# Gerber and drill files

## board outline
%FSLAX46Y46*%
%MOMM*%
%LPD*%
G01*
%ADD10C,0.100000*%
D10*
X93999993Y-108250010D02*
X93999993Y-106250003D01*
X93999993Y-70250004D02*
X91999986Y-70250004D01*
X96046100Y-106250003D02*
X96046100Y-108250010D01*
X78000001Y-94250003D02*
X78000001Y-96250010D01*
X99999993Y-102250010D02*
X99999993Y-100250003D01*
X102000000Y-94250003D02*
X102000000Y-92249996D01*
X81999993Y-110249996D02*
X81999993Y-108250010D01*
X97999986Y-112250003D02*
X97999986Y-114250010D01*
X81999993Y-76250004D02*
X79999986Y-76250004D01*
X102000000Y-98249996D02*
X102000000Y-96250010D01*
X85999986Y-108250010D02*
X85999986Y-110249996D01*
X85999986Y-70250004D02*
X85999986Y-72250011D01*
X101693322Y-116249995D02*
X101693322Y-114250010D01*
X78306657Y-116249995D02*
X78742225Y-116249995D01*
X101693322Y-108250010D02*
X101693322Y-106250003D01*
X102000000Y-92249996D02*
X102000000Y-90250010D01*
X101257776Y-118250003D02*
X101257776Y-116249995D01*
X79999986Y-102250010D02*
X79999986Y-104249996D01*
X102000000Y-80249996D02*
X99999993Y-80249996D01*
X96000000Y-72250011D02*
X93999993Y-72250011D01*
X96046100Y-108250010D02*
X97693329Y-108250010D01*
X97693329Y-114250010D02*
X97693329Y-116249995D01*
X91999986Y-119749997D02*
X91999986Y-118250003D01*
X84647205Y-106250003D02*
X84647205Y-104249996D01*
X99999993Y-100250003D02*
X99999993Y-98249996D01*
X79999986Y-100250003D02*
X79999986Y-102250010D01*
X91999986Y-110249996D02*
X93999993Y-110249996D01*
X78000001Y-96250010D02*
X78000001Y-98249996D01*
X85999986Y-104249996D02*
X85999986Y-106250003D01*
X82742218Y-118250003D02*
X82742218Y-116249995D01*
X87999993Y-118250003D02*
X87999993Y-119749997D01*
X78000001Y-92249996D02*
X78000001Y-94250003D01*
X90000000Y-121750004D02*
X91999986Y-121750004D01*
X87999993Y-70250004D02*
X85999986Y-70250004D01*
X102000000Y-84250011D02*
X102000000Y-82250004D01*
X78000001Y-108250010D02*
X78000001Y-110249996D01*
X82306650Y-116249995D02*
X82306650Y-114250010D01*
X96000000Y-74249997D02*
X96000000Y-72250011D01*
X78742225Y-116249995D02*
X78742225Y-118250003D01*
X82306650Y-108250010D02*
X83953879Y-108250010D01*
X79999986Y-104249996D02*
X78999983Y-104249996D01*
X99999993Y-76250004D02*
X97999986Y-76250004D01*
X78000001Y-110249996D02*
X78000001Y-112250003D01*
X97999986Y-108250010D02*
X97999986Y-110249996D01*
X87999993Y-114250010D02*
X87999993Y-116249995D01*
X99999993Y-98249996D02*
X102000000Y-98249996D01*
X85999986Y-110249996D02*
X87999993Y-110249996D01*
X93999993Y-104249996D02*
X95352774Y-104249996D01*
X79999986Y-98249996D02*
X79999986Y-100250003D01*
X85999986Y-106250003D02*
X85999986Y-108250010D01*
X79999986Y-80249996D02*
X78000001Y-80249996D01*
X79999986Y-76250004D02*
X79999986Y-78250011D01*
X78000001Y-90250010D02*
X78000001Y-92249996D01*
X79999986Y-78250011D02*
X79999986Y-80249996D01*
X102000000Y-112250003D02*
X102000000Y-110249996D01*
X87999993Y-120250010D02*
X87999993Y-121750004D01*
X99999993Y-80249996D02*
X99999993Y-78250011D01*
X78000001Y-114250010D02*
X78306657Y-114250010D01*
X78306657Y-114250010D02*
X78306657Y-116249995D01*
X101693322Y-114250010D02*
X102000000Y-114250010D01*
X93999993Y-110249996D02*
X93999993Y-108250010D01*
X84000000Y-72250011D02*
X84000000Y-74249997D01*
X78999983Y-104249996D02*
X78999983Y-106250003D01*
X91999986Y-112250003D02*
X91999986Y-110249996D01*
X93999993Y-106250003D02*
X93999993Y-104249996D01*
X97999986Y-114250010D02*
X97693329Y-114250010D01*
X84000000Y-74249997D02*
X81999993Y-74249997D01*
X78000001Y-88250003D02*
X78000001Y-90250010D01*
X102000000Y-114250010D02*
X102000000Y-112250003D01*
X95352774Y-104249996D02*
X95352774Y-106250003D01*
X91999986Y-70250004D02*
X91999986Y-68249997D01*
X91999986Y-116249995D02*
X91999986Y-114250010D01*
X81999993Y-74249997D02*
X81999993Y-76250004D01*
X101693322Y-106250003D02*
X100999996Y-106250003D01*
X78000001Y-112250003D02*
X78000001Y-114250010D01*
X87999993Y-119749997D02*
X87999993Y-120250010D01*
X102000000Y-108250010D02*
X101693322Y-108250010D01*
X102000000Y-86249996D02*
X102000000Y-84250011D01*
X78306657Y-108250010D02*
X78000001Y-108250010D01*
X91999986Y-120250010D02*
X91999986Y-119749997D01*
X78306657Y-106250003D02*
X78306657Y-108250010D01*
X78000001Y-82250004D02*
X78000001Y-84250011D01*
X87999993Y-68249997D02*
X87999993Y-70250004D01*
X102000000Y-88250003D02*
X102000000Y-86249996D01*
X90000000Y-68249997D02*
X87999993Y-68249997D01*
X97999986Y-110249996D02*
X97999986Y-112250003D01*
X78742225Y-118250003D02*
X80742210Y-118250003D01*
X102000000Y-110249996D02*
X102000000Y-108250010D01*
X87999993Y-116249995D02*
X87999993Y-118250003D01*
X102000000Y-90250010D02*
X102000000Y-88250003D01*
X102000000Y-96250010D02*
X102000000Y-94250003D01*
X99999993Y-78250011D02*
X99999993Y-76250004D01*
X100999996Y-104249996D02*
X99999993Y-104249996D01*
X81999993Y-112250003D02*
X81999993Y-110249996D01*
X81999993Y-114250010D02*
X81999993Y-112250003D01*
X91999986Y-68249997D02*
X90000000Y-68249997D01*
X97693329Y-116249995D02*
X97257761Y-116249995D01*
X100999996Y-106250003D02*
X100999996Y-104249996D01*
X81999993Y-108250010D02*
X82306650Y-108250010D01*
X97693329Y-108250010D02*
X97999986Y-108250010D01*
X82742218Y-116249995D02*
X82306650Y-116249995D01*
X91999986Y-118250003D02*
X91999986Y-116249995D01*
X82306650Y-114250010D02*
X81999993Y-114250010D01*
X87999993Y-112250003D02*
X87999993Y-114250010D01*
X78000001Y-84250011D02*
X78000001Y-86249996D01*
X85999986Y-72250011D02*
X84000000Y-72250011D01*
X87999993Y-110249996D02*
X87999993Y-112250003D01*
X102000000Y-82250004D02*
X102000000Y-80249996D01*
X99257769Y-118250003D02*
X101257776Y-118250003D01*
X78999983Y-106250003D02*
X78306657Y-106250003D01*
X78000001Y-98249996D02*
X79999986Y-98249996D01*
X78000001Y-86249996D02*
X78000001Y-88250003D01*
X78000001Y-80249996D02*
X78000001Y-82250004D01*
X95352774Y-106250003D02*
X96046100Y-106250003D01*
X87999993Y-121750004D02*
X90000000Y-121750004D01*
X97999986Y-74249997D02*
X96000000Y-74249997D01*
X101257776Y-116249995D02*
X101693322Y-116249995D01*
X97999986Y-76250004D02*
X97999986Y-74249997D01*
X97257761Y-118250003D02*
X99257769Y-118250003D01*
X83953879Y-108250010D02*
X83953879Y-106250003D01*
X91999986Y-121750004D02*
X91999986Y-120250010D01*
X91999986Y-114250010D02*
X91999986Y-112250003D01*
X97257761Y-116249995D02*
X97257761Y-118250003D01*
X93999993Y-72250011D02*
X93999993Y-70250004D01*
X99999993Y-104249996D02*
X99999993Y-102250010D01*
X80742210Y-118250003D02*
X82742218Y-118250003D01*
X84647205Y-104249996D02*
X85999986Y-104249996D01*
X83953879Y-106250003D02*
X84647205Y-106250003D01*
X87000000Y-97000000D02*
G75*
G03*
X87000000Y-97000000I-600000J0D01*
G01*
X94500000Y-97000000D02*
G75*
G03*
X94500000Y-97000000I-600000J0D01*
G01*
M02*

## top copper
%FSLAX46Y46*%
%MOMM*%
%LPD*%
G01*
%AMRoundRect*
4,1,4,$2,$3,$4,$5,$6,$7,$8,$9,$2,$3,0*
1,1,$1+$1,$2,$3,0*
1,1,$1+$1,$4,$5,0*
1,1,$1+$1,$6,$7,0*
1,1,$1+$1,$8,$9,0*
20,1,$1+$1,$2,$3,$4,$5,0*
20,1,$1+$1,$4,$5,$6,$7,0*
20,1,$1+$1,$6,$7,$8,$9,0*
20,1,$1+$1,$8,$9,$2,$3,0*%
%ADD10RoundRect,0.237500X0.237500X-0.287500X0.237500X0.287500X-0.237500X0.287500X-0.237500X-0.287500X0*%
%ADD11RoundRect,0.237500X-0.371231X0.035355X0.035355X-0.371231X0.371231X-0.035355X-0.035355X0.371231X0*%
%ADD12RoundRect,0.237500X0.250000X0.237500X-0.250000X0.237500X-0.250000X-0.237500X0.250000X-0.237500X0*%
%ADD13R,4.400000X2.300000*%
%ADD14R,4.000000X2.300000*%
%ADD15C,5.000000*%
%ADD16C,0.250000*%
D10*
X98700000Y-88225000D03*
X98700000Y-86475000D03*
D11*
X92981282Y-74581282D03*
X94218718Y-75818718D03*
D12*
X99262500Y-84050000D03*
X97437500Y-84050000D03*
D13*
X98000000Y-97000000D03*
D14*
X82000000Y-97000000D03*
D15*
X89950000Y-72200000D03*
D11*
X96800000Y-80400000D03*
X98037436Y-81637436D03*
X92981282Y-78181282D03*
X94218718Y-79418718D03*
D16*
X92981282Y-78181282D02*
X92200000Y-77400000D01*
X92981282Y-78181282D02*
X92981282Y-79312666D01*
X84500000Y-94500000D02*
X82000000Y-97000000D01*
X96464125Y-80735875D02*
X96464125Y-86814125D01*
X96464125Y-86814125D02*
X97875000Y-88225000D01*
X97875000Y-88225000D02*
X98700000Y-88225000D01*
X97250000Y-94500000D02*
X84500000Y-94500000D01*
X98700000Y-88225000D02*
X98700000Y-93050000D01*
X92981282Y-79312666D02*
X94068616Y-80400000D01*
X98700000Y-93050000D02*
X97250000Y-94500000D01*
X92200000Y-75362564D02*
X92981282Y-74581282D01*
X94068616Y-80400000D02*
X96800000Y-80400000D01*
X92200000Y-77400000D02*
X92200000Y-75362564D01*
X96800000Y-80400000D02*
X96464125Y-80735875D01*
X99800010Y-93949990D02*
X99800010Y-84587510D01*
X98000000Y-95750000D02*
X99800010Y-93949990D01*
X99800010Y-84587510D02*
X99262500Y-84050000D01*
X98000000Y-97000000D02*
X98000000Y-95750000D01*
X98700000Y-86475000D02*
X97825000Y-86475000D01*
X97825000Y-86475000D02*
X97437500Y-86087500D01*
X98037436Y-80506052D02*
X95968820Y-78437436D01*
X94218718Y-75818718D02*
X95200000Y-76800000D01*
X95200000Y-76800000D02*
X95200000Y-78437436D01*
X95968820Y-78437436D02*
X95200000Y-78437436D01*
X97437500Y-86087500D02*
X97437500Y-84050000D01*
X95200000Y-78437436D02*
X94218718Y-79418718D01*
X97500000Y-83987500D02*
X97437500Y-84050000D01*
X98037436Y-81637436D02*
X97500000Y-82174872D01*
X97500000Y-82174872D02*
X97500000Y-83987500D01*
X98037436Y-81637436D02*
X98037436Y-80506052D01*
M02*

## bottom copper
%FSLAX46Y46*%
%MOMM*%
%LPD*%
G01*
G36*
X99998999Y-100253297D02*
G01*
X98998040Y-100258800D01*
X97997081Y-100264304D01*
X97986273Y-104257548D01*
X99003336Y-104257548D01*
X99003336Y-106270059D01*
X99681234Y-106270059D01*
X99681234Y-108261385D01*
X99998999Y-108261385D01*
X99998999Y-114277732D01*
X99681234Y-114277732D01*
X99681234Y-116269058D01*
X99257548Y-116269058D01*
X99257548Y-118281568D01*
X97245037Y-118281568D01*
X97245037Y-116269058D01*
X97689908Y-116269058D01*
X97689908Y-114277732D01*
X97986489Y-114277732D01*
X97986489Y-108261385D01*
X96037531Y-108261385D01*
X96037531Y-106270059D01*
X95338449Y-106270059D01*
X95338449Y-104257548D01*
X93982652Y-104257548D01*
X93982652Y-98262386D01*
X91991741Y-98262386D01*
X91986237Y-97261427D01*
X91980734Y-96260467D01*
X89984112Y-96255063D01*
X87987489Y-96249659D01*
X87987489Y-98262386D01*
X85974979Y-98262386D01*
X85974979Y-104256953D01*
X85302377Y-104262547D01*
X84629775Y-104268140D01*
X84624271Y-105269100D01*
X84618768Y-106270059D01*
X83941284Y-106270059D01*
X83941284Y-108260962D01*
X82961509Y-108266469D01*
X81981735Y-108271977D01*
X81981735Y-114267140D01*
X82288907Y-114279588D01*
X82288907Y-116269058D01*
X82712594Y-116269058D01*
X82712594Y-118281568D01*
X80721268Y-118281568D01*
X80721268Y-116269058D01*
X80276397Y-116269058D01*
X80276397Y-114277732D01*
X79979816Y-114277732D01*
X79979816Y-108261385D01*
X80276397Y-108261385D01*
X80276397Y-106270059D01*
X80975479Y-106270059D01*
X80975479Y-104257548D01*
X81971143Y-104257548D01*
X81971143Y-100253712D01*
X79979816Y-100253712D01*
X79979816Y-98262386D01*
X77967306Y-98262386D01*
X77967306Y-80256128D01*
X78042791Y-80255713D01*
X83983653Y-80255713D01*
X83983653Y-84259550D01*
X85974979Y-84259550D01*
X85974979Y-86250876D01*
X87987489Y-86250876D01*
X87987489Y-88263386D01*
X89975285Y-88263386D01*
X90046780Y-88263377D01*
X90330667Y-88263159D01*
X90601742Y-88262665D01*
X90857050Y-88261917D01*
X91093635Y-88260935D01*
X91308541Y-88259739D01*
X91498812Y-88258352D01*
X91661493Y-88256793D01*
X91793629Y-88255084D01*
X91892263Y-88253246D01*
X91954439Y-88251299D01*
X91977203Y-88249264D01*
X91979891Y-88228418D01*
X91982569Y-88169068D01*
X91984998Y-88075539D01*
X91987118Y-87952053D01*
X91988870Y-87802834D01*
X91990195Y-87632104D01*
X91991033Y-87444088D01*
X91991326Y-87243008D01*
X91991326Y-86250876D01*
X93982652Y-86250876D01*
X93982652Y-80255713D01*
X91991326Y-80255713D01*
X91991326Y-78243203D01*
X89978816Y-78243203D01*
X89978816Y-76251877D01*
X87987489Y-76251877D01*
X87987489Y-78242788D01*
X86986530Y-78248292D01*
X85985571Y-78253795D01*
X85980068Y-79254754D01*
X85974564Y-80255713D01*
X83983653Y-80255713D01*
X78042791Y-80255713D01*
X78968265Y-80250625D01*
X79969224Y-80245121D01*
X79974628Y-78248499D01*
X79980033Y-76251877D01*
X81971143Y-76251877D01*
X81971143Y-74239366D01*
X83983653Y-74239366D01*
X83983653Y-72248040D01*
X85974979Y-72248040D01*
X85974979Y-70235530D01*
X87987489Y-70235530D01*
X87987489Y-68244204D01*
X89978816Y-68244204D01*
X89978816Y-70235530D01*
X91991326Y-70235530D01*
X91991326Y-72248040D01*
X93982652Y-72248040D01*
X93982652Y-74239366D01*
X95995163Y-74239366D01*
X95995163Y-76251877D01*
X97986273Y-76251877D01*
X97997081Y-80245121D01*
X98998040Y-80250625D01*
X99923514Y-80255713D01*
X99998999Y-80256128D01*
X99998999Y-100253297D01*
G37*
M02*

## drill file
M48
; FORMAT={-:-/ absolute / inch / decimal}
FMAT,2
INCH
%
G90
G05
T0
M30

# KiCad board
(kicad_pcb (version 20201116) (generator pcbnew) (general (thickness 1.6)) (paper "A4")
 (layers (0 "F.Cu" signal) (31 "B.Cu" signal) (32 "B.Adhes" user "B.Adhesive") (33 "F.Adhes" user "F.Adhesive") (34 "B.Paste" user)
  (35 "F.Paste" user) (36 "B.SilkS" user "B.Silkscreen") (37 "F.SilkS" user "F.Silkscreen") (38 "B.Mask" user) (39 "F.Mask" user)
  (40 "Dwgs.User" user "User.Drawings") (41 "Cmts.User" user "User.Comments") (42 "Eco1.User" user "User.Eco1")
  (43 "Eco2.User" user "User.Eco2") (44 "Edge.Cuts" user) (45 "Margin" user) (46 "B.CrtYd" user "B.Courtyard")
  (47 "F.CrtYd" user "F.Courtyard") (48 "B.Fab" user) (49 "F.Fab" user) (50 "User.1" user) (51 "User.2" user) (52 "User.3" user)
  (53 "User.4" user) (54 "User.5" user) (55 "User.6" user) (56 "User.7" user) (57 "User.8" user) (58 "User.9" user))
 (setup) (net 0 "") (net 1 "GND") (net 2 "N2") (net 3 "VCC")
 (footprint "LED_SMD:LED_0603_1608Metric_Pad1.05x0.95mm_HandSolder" (layer "F.Cu") (at 98.7 87.35 90)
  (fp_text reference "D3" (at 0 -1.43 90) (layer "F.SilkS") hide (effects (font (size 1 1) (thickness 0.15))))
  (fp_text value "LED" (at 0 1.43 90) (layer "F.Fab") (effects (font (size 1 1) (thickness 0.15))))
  (pad "1" smd roundrect (at -0.875 0 90) (size 1.05 0.95) (layers "F.Cu" "F.Paste" "F.Mask") (roundrect_rratio 0.25) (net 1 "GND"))
  (pad "2" smd roundrect (at 0.875 0 90) (size 1.05 0.95) (layers "F.Cu" "F.Paste" "F.Mask") (roundrect_rratio 0.25) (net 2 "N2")))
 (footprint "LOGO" (layer "F.Cu") (at 82.05 87.7)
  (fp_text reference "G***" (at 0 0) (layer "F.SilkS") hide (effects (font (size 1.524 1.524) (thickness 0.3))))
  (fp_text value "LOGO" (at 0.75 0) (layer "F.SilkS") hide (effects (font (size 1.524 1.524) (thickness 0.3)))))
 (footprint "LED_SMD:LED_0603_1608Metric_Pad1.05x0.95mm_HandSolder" (layer "F.Cu") (at 93.6 75.2 -45)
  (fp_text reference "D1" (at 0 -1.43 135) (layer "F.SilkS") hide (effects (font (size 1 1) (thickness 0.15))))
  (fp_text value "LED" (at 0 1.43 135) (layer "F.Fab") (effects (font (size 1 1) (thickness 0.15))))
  (pad "1" smd roundrect (at -0.875 0 315) (size 1.05 0.95) (layers "F.Cu" "F.Paste" "F.Mask") (roundrect_rratio 0.25) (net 1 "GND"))
  (pad "2" smd roundrect (at 0.875 0 315) (size 1.05 0.95) (layers "F.Cu" "F.Paste" "F.Mask") (roundrect_rratio 0.25) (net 2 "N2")))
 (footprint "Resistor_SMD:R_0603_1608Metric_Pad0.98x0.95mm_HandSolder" (layer "F.Cu") (at 98.35 84.05 180)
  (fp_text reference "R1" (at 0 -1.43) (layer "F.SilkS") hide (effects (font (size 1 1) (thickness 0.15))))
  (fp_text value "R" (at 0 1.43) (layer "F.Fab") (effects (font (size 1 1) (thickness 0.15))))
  (pad "1" smd roundrect (at -0.9125 0 180) (size 0.975 0.95) (layers "F.Cu" "F.Paste" "F.Mask") (roundrect_rratio 0.25) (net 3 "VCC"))
  (pad "2" smd roundrect (at 0.9125 0 180) (size 0.975 0.95) (layers "F.Cu" "F.Paste" "F.Mask") (roundrect_rratio 0.25) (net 2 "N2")))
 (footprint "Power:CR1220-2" (layer "F.Cu") (at 90 97 90)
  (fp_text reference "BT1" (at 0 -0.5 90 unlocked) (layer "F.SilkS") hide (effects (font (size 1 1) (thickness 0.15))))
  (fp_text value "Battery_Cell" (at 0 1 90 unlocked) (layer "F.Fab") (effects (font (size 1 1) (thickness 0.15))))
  (fp_circle (center 0 -3.6) (end 0.6 -3.6) (layer "Edge.Cuts") (width 0.1) (fill none))
  (fp_circle (center 0 3.9) (end 0.6 3.9) (layer "Edge.Cuts") (width 0.1) (fill none))
  (pad "1" smd rect (at 0 8 90) (size 2.3 4.4) (layers "F.Cu" "F.Paste" "F.Mask") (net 3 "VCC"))
  (pad "2" smd rect (at 0 -8 90) (size 2.3 4) (layers "F.Cu" "F.Paste" "F.Mask") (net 1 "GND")))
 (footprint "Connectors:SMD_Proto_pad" (layer "F.Cu") (at 89.95 72.2)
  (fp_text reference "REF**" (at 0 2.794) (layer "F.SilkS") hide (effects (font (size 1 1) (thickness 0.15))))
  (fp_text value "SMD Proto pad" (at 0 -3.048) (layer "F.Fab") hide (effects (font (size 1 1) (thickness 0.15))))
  (pad "1" smd circle (at 0 0) (size 5 5) (layers "F.Cu" "F.Mask")))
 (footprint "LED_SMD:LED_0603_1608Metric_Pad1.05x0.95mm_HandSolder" (layer "F.Cu") (at 97.418718 81.018718 -45)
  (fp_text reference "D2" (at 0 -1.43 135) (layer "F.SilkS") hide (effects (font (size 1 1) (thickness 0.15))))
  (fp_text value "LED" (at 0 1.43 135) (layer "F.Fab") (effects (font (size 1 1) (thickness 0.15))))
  (pad "1" smd roundrect (at -0.875 0 315) (size 1.05 0.95) (layers "F.Cu" "F.Paste" "F.Mask") (roundrect_rratio 0.25) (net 1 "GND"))
  (pad "2" smd roundrect (at 0.875 0 315) (size 1.05 0.95) (layers "F.Cu" "F.Paste" "F.Mask") (roundrect_rratio 0.25) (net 2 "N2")))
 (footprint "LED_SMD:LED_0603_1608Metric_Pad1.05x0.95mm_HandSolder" (layer "F.Cu") (at 93.6 78.8 -45)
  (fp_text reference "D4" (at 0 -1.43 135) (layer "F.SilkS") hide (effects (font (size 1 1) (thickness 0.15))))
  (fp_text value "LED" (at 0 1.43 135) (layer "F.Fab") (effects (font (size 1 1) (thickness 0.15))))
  (pad "1" smd roundrect (at -0.875 0 315) (size 1.05 0.95) (layers "F.Cu" "F.Paste" "F.Mask") (roundrect_rratio 0.25) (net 1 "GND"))
  (pad "2" smd roundrect (at 0.875 0 315) (size 1.05 0.95) (layers "F.Cu" "F.Paste" "F.Mask") (roundrect_rratio 0.25) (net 2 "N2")))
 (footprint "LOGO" (layer "B.Cu") (at 90 95 180)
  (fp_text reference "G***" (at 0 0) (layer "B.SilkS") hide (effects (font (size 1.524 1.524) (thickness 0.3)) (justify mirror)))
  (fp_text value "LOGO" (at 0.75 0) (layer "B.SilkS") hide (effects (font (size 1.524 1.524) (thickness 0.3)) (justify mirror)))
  (fp_poly
   (pts (xy 2.012511 24.76447) (xy 4.025021 24.76447) (xy 4.025021 22.75196) (xy 6.016347 22.75196) (xy 6.016347 20.760634)
    (xy 8.028857 20.760634) (xy 8.028857 18.748123) (xy 10.019967 18.748123) (xy 10.025372 16.751501) (xy 10.030776 14.754879)
    (xy 11.031735 14.749375) (xy 12.032694 14.743872) (xy 12.032694 -3.262386) (xy 10.020184 -3.262386) (xy 10.020184 -5.253712)
    (xy 8.028857 -5.253712) (xy 8.028857 -9.257548) (xy 9.024521 -9.257548) (xy 9.024521 -11.270059) (xy 9.723603 -11.270059)
    (xy 9.723603 -13.261385) (xy 10.020184 -13.261385) (xy 10.020184 -19.277732) (xy 9.723603 -19.277732) (xy 9.723603 -21.269058)
    (xy 9.278732 -21.269058) (xy 9.278732 -23.281568) (xy 7.287406 -23.281568) (xy 7.287406 -21.269058) (xy 7.711093 -21.269058)
    (xy 7.711093 -19.279588) (xy 8.018265 -19.26714) (xy 8.018265 -13.271977) (xy 7.038491 -13.266469) (xy 6.058716 -13.260962)
    (xy 6.058716 -11.270059) (xy 5.381232 -11.270059) (xy 5.375729 -10.2691) (xy 5.370225 -9.26814) (xy 4.697623 -9.262547)
    (xy 4.025021 -9.256953) (xy 4.025021 -3.262386) (xy 2.012511 -3.262386) (xy 2.012511 -1.249659) (xy 0.015888 -1.255063)
    (xy -1.980734 -1.260467) (xy -1.986237 -2.261427) (xy -1.991741 -3.262386) (xy -3.982652 -3.262386) (xy -3.982652 -9.257548)
    (xy -5.338449 -9.257548) (xy -5.338449 -11.270059) (xy -6.037531 -11.270059) (xy -6.037531 -13.261385) (xy -7.986489 -13.261385)
    (xy -7.986489 -19.277732) (xy -7.689908 -19.277732) (xy -7.689908 -21.269058) (xy -7.245037 -21.269058) (xy -7.245037 -23.281568)
    (xy -9.257548 -23.281568) (xy -9.257548 -21.269058) (xy -9.681234 -21.269058) (xy -9.681234 -19.277732) (xy -9.998999 -19.277732)
    (xy -9.998999 -13.261385) (xy -9.681234 -13.261385) (xy -9.681234 -11.270059) (xy -9.003336 -11.270059) (xy -9.003336 -9.257548)
    (xy -7.986273 -9.257548) (xy -7.997081 -5.264304) (xy -8.99804 -5.2588) (xy -9.998999 -5.253297) (xy -9.998999 14.743872)
    (xy -9.923514 14.744287) (xy -3.982652 14.744287) (xy -3.982652 8.749124) (xy -1.991326 8.749124) (xy -1.991326 7.756992)
    (xy -1.991033 7.555912) (xy -1.990195 7.367896) (xy -1.98887 7.197166) (xy -1.987118 7.047947) (xy -1.984998 6.924461)
    (xy -1.982569 6.830932) (xy -1.979891 6.771582) (xy -1.977203 6.750736) (xy -1.954439 6.748701) (xy -1.892263 6.746754)
    (xy -1.793629 6.744916) (xy -1.661493 6.743207) (xy -1.498812 6.741648) (xy -1.308541 6.740261) (xy -1.093635 6.739065)
    (xy -0.85705 6.738083) (xy -0.601742 6.737335) (xy -0.330667 6.736841) (xy -0.04678 6.736623) (xy 0.024715 6.736614)
    (xy 2.012511 6.736614) (xy 2.012511 8.749124) (xy 4.025021 8.749124) (xy 4.025021 10.74045) (xy 6.016347 10.74045)
    (xy 6.016347 14.744287) (xy 4.025436 14.744287) (xy 4.019932 15.745246) (xy 4.014429 16.746205) (xy 3.01347 16.751708)
    (xy 2.012511 16.757212) (xy 2.012511 18.748123) (xy 0.021184 18.748123) (xy 0.021184 16.756797) (xy -1.991326 16.756797)
    (xy -1.991326 14.744287) (xy -3.982652 14.744287) (xy -9.923514 14.744287) (xy -8.99804 14.749375) (xy -7.997081 14.754879)
    (xy -7.986273 18.748123) (xy -5.995163 18.748123) (xy -5.995163 20.760634) (xy -3.982652 20.760634) (xy -3.982652 22.75196)
    (xy -1.991326 22.75196) (xy -1.991326 24.76447) (xy 0.021184 24.76447) (xy 0.021184 26.755796) (xy 2.012511 26.755796))
   (layer "B.Cu") (width 0) (fill solid)))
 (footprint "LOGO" (layer "B.Cu") (at 90 95 180)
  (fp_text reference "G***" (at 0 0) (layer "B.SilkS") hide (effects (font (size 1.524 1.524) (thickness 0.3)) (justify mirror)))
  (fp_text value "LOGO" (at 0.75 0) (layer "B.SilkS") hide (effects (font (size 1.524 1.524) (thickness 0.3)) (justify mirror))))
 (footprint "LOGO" (layer "B.Cu") (at 90 95 180)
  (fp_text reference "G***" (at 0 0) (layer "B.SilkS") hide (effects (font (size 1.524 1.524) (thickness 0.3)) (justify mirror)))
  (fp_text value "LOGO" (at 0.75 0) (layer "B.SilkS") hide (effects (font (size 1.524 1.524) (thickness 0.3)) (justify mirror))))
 (gr_line (start 93.999993 108.25001) (end 93.999993 106.250003) (layer "Edge.Cuts") (width 0.1))
 (gr_line (start 93.999993 70.250004) (end 91.999986 70.250004) (layer "Edge.Cuts") (width 0.1))
 (gr_line (start 96.0461 106.250003) (end 96.0461 108.25001) (layer "Edge.Cuts") (width 0.1))
 (gr_line (start 78.000001 94.250003) (end 78.000001 96.25001) (layer "Edge.Cuts") (width 0.1))
 (gr_line (start 99.999993 102.25001) (end 99.999993 100.250003) (layer "Edge.Cuts") (width 0.1))
 (gr_line (start 102 94.250003) (end 102 92.249996) (layer "Edge.Cuts") (width 0.1))
 (gr_line (start 81.999993 110.249996) (end 81.999993 108.25001) (layer "Edge.Cuts") (width 0.1))
 (gr_line (start 97.999986 112.250003) (end 97.999986 114.25001) (layer "Edge.Cuts") (width 0.1))
 (gr_line (start 81.999993 76.250004) (end 79.999986 76.250004) (layer "Edge.Cuts") (width 0.1))
 (gr_line (start 102 98.249996) (end 102 96.25001) (layer "Edge.Cuts") (width 0.1))
 (gr_line (start 85.999986 108.25001) (end 85.999986 110.249996) (layer "Edge.Cuts") (width 0.1))
 (gr_line (start 85.999986 70.250004) (end 85.999986 72.250011) (layer "Edge.Cuts") (width 0.1))
 (gr_line (start 101.693322 116.249995) (end 101.693322 114.25001) (layer "Edge.Cuts") (width 0.1))
 (gr_line (start 78.306657 116.249995) (end 78.742225 116.249995) (layer "Edge.Cuts") (width 0.1))
 (gr_line (start 101.693322 108.25001) (end 101.693322 106.250003) (layer "Edge.Cuts") (width 0.1))
 (gr_line (start 102 92.249996) (end 102 90.25001) (layer "Edge.Cuts") (width 0.1))
 (gr_line (start 101.257776 118.250003) (end 101.257776 116.249995) (layer "Edge.Cuts") (width 0.1))
 (gr_line (start 79.999986 102.25001) (end 79.999986 104.249996) (layer "Edge.Cuts") (width 0.1))
 (gr_line (start 102 80.249996) (end 99.999993 80.249996) (layer "Edge.Cuts") (width 0.1))
 (gr_line (start 96 72.250011) (end 93.999993 72.250011) (layer "Edge.Cuts") (width 0.1))
 (gr_line (start 96.0461 108.25001) (end 97.693329 108.25001) (layer "Edge.Cuts") (width 0.1))
 (gr_line (start 97.693329 114.25001) (end 97.693329 116.249995) (layer "Edge.Cuts") (width 0.1))
 (gr_line (start 91.999986 119.749997) (end 91.999986 118.250003) (layer "Edge.Cuts") (width 0.1))
 (gr_line (start 84.647205 106.250003) (end 84.647205 104.249996) (layer "Edge.Cuts") (width 0.1))
 (gr_line (start 99.999993 100.250003) (end 99.999993 98.249996) (layer "Edge.Cuts") (width 0.1))
 (gr_line (start 79.999986 100.250003) (end 79.999986 102.25001) (layer "Edge.Cuts") (width 0.1))
 (gr_line (start 91.999986 110.249996) (end 93.999993 110.249996) (layer "Edge.Cuts") (width 0.1))
 (gr_line (start 78.000001 96.25001) (end 78.000001 98.249996) (layer "Edge.Cuts") (width 0.1))
 (gr_line (start 85.999986 104.249996) (end 85.999986 106.250003) (layer "Edge.Cuts") (width 0.1))
 (gr_line (start 82.742218 118.250003) (end 82.742218 116.249995) (layer "Edge.Cuts") (width 0.1))
 (gr_line (start 87.999993 118.250003) (end 87.999993 119.749997) (layer "Edge.Cuts") (width 0.1))
 (gr_line (start 78.000001 92.249996) (end 78.000001 94.250003) (layer "Edge.Cuts") (width 0.1))
 (gr_line (start 90 121.750004) (end 91.999986 121.750004) (layer "Edge.Cuts") (width 0.1))
 (gr_line (start 87.999993 70.250004) (end 85.999986 70.250004) (layer "Edge.Cuts") (width 0.1))
 (gr_line (start 102 84.250011) (end 102 82.250004) (layer "Edge.Cuts") (width 0.1))
 (gr_line (start 78.000001 108.25001) (end 78.000001 110.249996) (layer "Edge.Cuts") (width 0.1))
 (gr_line (start 82.30665 116.249995) (end 82.30665 114.25001) (layer "Edge.Cuts") (width 0.1))
 (gr_line (start 96 74.249997) (end 96 72.250011) (layer "Edge.Cuts") (width 0.1))
 (gr_line (start 78.742225 116.249995) (end 78.742225 118.250003) (layer "Edge.Cuts") (width 0.1))
 (gr_line (start 82.30665 108.25001) (end 83.953879 108.25001) (layer "Edge.Cuts") (width 0.1))
 (gr_line (start 79.999986 104.249996) (end 78.999983 104.249996) (layer "Edge.Cuts") (width 0.1))
 (gr_line (start 99.999993 76.250004) (end 97.999986 76.250004) (layer "Edge.Cuts") (width 0.1))
 (gr_line (start 78.000001 110.249996) (end 78.000001 112.250003) (layer "Edge.Cuts") (width 0.1))
 (gr_line (start 97.999986 108.25001) (end 97.999986 110.249996) (layer "Edge.Cuts") (width 0.1))
 (gr_line (start 87.999993 114.25001) (end 87.999993 116.249995) (layer "Edge.Cuts") (width 0.1))
 (gr_line (start 99.999993 98.249996) (end 102 98.249996) (layer "Edge.Cuts") (width 0.1))
 (gr_line (start 85.999986 110.249996) (end 87.999993 110.249996) (layer "Edge.Cuts") (width 0.1))
 (gr_line (start 93.999993 104.249996) (end 95.352774 104.249996) (layer "Edge.Cuts") (width 0.1))
 (gr_line (start 79.999986 98.249996) (end 79.999986 100.250003) (layer "Edge.Cuts") (width 0.1))
 (gr_line (start 85.999986 106.250003) (end 85.999986 108.25001) (layer "Edge.Cuts") (width 0.1))
 (gr_line (start 79.999986 80.249996) (end 78.000001 80.249996) (layer "Edge.Cuts") (width 0.1))
 (gr_line (start 79.999986 76.250004) (end 79.999986 78.250011) (layer "Edge.Cuts") (width 0.1))
 (gr_line (start 78.000001 90.25001) (end 78.000001 92.249996) (layer "Edge.Cuts") (width 0.1))
 (gr_line (start 79.999986 78.250011) (end 79.999986 80.249996) (layer "Edge.Cuts") (width 0.1))
 (gr_line (start 102 112.250003) (end 102 110.249996) (layer "Edge.Cuts") (width 0.1))
 (gr_line (start 87.999993 120.25001) (end 87.999993 121.750004) (layer "Edge.Cuts") (width 0.1))
 (gr_line (start 99.999993 80.249996) (end 99.999993 78.250011) (layer "Edge.Cuts") (width 0.1))
 (gr_line (start 78.000001 114.25001) (end 78.306657 114.25001) (layer "Edge.Cuts") (width 0.1))
 (gr_line (start 78.306657 114.25001) (end 78.306657 116.249995) (layer "Edge.Cuts") (width 0.1))
 (gr_line (start 101.693322 114.25001) (end 102 114.25001) (layer "Edge.Cuts") (width 0.1))
 (gr_line (start 93.999993 110.249996) (end 93.999993 108.25001) (layer "Edge.Cuts") (width 0.1))
 (gr_line (start 84 72.250011) (end 84 74.249997) (layer "Edge.Cuts") (width 0.1))
 (gr_line (start 78.999983 104.249996) (end 78.999983 106.250003) (layer "Edge.Cuts") (width 0.1))
 (gr_line (start 91.999986 112.250003) (end 91.999986 110.249996) (layer "Edge.Cuts") (width 0.1))
 (gr_line (start 93.999993 106.250003) (end 93.999993 104.249996) (layer "Edge.Cuts") (width 0.1))
 (gr_line (start 97.999986 114.25001) (end 97.693329 114.25001) (layer "Edge.Cuts") (width 0.1))
 (gr_line (start 84 74.249997) (end 81.999993 74.249997) (layer "Edge.Cuts") (width 0.1))
 (gr_line (start 78.000001 88.250003) (end 78.000001 90.25001) (layer "Edge.Cuts") (width 0.1))
 (gr_line (start 102 114.25001) (end 102 112.250003) (layer "Edge.Cuts") (width 0.1))
 (gr_line (start 95.352774 104.249996) (end 95.352774 106.250003) (layer "Edge.Cuts") (width 0.1))
 (gr_line (start 91.999986 70.250004) (end 91.999986 68.249997) (layer "Edge.Cuts") (width 0.1))
 (gr_line (start 91.999986 116.249995) (end 91.999986 114.25001) (layer "Edge.Cuts") (width 0.1))
 (gr_line (start 81.999993 74.249997) (end 81.999993 76.250004) (layer "Edge.Cuts") (width 0.1))
 (gr_line (start 101.693322 106.250003) (end 100.999996 106.250003) (layer "Edge.Cuts") (width 0.1))
 (gr_line (start 78.000001 112.250003) (end 78.000001 114.25001) (layer "Edge.Cuts") (width 0.1))
 (gr_line (start 87.999993 119.749997) (end 87.999993 120.25001) (layer "Edge.Cuts") (width 0.1))
 (gr_line (start 102 108.25001) (end 101.693322 108.25001) (layer "Edge.Cuts") (width 0.1))
 (gr_line (start 102 86.249996) (end 102 84.250011) (layer "Edge.Cuts") (width 0.1))
 (gr_line (start 78.306657 108.25001) (end 78.000001 108.25001) (layer "Edge.Cuts") (width 0.1))
 (gr_line (start 91.999986 120.25001) (end 91.999986 119.749997) (layer "Edge.Cuts") (width 0.1))
 (gr_line (start 78.306657 106.250003) (end 78.306657 108.25001) (layer "Edge.Cuts") (width 0.1))
 (gr_line (start 78.000001 82.250004) (end 78.000001 84.250011) (layer "Edge.Cuts") (width 0.1))
 (gr_line (start 87.999993 68.249997) (end 87.999993 70.250004) (layer "Edge.Cuts") (width 0.1))
 (gr_line (start 102 88.250003) (end 102 86.249996) (layer "Edge.Cuts") (width 0.1))
 (gr_line (start 90 68.249997) (end 87.999993 68.249997) (layer "Edge.Cuts") (width 0.1))
 (gr_line (start 97.999986 110.249996) (end 97.999986 112.250003) (layer "Edge.Cuts") (width 0.1))
 (gr_line (start 78.742225 118.250003) (end 80.74221 118.250003) (layer "Edge.Cuts") (width 0.1))
 (gr_line (start 102 110.249996) (end 102 108.25001) (layer "Edge.Cuts") (width 0.1))
 (gr_line (start 87.999993 116.249995) (end 87.999993 118.250003) (layer "Edge.Cuts") (width 0.1))
 (gr_line (start 102 90.25001) (end 102 88.250003) (layer "Edge.Cuts") (width 0.1))
 (gr_line (start 102 96.25001) (end 102 94.250003) (layer "Edge.Cuts") (width 0.1))
 (gr_line (start 99.999993 78.250011) (end 99.999993 76.250004) (layer "Edge.Cuts") (width 0.1))
 (gr_line (start 100.999996 104.249996) (end 99.999993 104.249996) (layer "Edge.Cuts") (width 0.1))
 (gr_line (start 81.999993 112.250003) (end 81.999993 110.249996) (layer "Edge.Cuts") (width 0.1))
 (gr_line (start 81.999993 114.25001) (end 81.999993 112.250003) (layer "Edge.Cuts") (width 0.1))
 (gr_line (start 91.999986 68.249997) (end 90 68.249997) (layer "Edge.Cuts") (width 0.1))
 (gr_line (start 97.693329 116.249995) (end 97.257761 116.249995) (layer "Edge.Cuts") (width 0.1))
 (gr_line (start 100.999996 106.250003) (end 100.999996 104.249996) (layer "Edge.Cuts") (width 0.1))
 (gr_line (start 81.999993 108.25001) (end 82.30665 108.25001) (layer "Edge.Cuts") (width 0.1))
 (gr_line (start 97.693329 108.25001) (end 97.999986 108.25001) (layer "Edge.Cuts") (width 0.1))
 (gr_line (start 82.742218 116.249995) (end 82.30665 116.249995) (layer "Edge.Cuts") (width 0.1))
 (gr_line (start 91.999986 118.250003) (end 91.999986 116.249995) (layer "Edge.Cuts") (width 0.1))
 (gr_line (start 82.30665 114.25001) (end 81.999993 114.25001) (layer "Edge.Cuts") (width 0.1))
 (gr_line (start 87.999993 112.250003) (end 87.999993 114.25001) (layer "Edge.Cuts") (width 0.1))
 (gr_line (start 78.000001 84.250011) (end 78.000001 86.249996) (layer "Edge.Cuts") (width 0.1))
 (gr_line (start 85.999986 72.250011) (end 84 72.250011) (layer "Edge.Cuts") (width 0.1))
 (gr_line (start 87.999993 110.249996) (end 87.999993 112.250003) (layer "Edge.Cuts") (width 0.1))
 (gr_line (start 102 82.250004) (end 102 80.249996) (layer "Edge.Cuts") (width 0.1))
 (gr_line (start 99.257769 118.250003) (end 101.257776 118.250003) (layer "Edge.Cuts") (width 0.1))
 (gr_line (start 78.999983 106.250003) (end 78.306657 106.250003) (layer "Edge.Cuts") (width 0.1))
 (gr_line (start 78.000001 98.249996) (end 79.999986 98.249996) (layer "Edge.Cuts") (width 0.1))
 (gr_line (start 78.000001 86.249996) (end 78.000001 88.250003) (layer "Edge.Cuts") (width 0.1))
 (gr_line (start 78.000001 80.249996) (end 78.000001 82.250004) (layer "Edge.Cuts") (width 0.1))
 (gr_line (start 95.352774 106.250003) (end 96.0461 106.250003) (layer "Edge.Cuts") (width 0.1))
 (gr_line (start 87.999993 121.750004) (end 90 121.750004) (layer "Edge.Cuts") (width 0.1))
 (gr_line (start 97.999986 74.249997) (end 96 74.249997) (layer "Edge.Cuts") (width 0.1))
 (gr_line (start 101.257776 116.249995) (end 101.693322 116.249995) (layer "Edge.Cuts") (width 0.1))
 (gr_line (start 97.999986 76.250004) (end 97.999986 74.249997) (layer "Edge.Cuts") (width 0.1))
 (gr_line (start 97.257761 118.250003) (end 99.257769 118.250003) (layer "Edge.Cuts") (width 0.1))
 (gr_line (start 83.953879 108.25001) (end 83.953879 106.250003) (layer "Edge.Cuts") (width 0.1))
 (gr_line (start 91.999986 121.750004) (end 91.999986 120.25001) (layer "Edge.Cuts") (width 0.1))
 (gr_line (start 91.999986 114.25001) (end 91.999986 112.250003) (layer "Edge.Cuts") (width 0.1))
 (gr_line (start 97.257761 116.249995) (end 97.257761 118.250003) (layer "Edge.Cuts") (width 0.1))
 (gr_line (start 93.999993 72.250011) (end 93.999993 70.250004) (layer "Edge.Cuts") (width 0.1))
 (gr_line (start 99.999993 104.249996) (end 99.999993 102.25001) (layer "Edge.Cuts") (width 0.1))
 (gr_line (start 80.74221 118.250003) (end 82.742218 118.250003) (layer "Edge.Cuts") (width 0.1))
 (gr_line (start 84.647205 104.249996) (end 85.999986 104.249996) (layer "Edge.Cuts") (width 0.1))
 (gr_line (start 83.953879 106.250003) (end 84.647205 106.250003) (layer "Edge.Cuts") (width 0.1))
 (segment (start 92.981282 78.181282) (end 92.2 77.4) (width 0.25) (layer "F.Cu") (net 1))
 (segment (start 92.981282 78.181282) (end 92.981282 79.312666) (width 0.25) (layer "F.Cu") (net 1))
 (segment (start 84.5 94.5) (end 82 97) (width 0.25) (layer "F.Cu") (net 1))
 (segment (start 96.464125 80.735875) (end 96.464125 86.814125) (width 0.25) (layer "F.Cu") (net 1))
 (segment (start 96.464125 86.814125) (end 97.875 88.225) (width 0.25) (layer "F.Cu") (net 1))
 (segment (start 97.875 88.225) (end 98.7 88.225) (width 0.25) (layer "F.Cu") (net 1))
 (segment (start 97.25 94.5) (end 84.5 94.5) (width 0.25) (layer "F.Cu") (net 1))
 (segment (start 98.7 88.225) (end 98.7 93.05) (width 0.25) (layer "F.Cu") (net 1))
 (segment (start 92.981282 79.312666) (end 94.068616 80.4) (width 0.25) (layer "F.Cu") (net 1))
 (segment (start 98.7 93.05) (end 97.25 94.5) (width 0.25) (layer "F.Cu") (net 1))
 (segment (start 92.2 75.362564) (end 92.981282 74.581282) (width 0.25) (layer "F.Cu") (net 1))
 (segment (start 94.068616 80.4) (end 96.8 80.4) (width 0.25) (layer "F.Cu") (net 1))
 (segment (start 92.2 77.4) (end 92.2 75.362564) (width 0.25) (layer "F.Cu") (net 1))
 (segment (start 96.8 80.4) (end 96.464125 80.735875) (width 0.25) (layer "F.Cu") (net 1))
 (segment (start 99.80001 93.94999) (end 99.80001 84.58751) (width 0.25) (layer "F.Cu") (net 3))
 (segment (start 98 95.75) (end 99.80001 93.94999) (width 0.25) (layer "F.Cu") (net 3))
 (segment (start 99.80001 84.58751) (end 99.2625 84.05) (width 0.25) (layer "F.Cu") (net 3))
 (segment (start 98 97) (end 98 95.75) (width 0.25) (layer "F.Cu") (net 3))
 (segment (start 98.7 86.475) (end 97.825 86.475) (width 0.25) (layer "F.Cu") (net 2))
 (segment (start 97.825 86.475) (end 97.4375 86.0875) (width 0.25) (layer "F.Cu") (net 2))
 (segment (start 98.037436 80.506052) (end 95.96882 78.437436) (width 0.25) (layer "F.Cu") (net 2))
 (segment (start 94.218718 75.818718) (end 95.2 76.8) (width 0.25) (layer "F.Cu") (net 2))
 (segment (start 95.2 76.8) (end 95.2 78.437436) (width 0.25) (layer "F.Cu") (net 2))
 (segment (start 95.96882 78.437436) (end 95.2 78.437436) (width 0.25) (layer "F.Cu") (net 2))
 (segment (start 97.4375 86.0875) (end 97.4375 84.05) (width 0.25) (layer "F.Cu") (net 2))
 (segment (start 95.2 78.437436) (end 94.218718 79.418718) (width 0.25) (layer "F.Cu") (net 2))
 (segment (start 97.5 83.9875) (end 97.4375 84.05) (width 0.25) (layer "F.Cu") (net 2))
 (segment (start 98.037436 81.637436) (end 97.5 82.174872) (width 0.25) (layer "F.Cu") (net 2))
 (segment (start 97.5 82.174872) (end 97.5 83.9875) (width 0.25) (layer "F.Cu") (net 2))
 (segment (start 98.037436 81.637436) (end 98.037436 80.506052) (width 0.25) (layer "F.Cu") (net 2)))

